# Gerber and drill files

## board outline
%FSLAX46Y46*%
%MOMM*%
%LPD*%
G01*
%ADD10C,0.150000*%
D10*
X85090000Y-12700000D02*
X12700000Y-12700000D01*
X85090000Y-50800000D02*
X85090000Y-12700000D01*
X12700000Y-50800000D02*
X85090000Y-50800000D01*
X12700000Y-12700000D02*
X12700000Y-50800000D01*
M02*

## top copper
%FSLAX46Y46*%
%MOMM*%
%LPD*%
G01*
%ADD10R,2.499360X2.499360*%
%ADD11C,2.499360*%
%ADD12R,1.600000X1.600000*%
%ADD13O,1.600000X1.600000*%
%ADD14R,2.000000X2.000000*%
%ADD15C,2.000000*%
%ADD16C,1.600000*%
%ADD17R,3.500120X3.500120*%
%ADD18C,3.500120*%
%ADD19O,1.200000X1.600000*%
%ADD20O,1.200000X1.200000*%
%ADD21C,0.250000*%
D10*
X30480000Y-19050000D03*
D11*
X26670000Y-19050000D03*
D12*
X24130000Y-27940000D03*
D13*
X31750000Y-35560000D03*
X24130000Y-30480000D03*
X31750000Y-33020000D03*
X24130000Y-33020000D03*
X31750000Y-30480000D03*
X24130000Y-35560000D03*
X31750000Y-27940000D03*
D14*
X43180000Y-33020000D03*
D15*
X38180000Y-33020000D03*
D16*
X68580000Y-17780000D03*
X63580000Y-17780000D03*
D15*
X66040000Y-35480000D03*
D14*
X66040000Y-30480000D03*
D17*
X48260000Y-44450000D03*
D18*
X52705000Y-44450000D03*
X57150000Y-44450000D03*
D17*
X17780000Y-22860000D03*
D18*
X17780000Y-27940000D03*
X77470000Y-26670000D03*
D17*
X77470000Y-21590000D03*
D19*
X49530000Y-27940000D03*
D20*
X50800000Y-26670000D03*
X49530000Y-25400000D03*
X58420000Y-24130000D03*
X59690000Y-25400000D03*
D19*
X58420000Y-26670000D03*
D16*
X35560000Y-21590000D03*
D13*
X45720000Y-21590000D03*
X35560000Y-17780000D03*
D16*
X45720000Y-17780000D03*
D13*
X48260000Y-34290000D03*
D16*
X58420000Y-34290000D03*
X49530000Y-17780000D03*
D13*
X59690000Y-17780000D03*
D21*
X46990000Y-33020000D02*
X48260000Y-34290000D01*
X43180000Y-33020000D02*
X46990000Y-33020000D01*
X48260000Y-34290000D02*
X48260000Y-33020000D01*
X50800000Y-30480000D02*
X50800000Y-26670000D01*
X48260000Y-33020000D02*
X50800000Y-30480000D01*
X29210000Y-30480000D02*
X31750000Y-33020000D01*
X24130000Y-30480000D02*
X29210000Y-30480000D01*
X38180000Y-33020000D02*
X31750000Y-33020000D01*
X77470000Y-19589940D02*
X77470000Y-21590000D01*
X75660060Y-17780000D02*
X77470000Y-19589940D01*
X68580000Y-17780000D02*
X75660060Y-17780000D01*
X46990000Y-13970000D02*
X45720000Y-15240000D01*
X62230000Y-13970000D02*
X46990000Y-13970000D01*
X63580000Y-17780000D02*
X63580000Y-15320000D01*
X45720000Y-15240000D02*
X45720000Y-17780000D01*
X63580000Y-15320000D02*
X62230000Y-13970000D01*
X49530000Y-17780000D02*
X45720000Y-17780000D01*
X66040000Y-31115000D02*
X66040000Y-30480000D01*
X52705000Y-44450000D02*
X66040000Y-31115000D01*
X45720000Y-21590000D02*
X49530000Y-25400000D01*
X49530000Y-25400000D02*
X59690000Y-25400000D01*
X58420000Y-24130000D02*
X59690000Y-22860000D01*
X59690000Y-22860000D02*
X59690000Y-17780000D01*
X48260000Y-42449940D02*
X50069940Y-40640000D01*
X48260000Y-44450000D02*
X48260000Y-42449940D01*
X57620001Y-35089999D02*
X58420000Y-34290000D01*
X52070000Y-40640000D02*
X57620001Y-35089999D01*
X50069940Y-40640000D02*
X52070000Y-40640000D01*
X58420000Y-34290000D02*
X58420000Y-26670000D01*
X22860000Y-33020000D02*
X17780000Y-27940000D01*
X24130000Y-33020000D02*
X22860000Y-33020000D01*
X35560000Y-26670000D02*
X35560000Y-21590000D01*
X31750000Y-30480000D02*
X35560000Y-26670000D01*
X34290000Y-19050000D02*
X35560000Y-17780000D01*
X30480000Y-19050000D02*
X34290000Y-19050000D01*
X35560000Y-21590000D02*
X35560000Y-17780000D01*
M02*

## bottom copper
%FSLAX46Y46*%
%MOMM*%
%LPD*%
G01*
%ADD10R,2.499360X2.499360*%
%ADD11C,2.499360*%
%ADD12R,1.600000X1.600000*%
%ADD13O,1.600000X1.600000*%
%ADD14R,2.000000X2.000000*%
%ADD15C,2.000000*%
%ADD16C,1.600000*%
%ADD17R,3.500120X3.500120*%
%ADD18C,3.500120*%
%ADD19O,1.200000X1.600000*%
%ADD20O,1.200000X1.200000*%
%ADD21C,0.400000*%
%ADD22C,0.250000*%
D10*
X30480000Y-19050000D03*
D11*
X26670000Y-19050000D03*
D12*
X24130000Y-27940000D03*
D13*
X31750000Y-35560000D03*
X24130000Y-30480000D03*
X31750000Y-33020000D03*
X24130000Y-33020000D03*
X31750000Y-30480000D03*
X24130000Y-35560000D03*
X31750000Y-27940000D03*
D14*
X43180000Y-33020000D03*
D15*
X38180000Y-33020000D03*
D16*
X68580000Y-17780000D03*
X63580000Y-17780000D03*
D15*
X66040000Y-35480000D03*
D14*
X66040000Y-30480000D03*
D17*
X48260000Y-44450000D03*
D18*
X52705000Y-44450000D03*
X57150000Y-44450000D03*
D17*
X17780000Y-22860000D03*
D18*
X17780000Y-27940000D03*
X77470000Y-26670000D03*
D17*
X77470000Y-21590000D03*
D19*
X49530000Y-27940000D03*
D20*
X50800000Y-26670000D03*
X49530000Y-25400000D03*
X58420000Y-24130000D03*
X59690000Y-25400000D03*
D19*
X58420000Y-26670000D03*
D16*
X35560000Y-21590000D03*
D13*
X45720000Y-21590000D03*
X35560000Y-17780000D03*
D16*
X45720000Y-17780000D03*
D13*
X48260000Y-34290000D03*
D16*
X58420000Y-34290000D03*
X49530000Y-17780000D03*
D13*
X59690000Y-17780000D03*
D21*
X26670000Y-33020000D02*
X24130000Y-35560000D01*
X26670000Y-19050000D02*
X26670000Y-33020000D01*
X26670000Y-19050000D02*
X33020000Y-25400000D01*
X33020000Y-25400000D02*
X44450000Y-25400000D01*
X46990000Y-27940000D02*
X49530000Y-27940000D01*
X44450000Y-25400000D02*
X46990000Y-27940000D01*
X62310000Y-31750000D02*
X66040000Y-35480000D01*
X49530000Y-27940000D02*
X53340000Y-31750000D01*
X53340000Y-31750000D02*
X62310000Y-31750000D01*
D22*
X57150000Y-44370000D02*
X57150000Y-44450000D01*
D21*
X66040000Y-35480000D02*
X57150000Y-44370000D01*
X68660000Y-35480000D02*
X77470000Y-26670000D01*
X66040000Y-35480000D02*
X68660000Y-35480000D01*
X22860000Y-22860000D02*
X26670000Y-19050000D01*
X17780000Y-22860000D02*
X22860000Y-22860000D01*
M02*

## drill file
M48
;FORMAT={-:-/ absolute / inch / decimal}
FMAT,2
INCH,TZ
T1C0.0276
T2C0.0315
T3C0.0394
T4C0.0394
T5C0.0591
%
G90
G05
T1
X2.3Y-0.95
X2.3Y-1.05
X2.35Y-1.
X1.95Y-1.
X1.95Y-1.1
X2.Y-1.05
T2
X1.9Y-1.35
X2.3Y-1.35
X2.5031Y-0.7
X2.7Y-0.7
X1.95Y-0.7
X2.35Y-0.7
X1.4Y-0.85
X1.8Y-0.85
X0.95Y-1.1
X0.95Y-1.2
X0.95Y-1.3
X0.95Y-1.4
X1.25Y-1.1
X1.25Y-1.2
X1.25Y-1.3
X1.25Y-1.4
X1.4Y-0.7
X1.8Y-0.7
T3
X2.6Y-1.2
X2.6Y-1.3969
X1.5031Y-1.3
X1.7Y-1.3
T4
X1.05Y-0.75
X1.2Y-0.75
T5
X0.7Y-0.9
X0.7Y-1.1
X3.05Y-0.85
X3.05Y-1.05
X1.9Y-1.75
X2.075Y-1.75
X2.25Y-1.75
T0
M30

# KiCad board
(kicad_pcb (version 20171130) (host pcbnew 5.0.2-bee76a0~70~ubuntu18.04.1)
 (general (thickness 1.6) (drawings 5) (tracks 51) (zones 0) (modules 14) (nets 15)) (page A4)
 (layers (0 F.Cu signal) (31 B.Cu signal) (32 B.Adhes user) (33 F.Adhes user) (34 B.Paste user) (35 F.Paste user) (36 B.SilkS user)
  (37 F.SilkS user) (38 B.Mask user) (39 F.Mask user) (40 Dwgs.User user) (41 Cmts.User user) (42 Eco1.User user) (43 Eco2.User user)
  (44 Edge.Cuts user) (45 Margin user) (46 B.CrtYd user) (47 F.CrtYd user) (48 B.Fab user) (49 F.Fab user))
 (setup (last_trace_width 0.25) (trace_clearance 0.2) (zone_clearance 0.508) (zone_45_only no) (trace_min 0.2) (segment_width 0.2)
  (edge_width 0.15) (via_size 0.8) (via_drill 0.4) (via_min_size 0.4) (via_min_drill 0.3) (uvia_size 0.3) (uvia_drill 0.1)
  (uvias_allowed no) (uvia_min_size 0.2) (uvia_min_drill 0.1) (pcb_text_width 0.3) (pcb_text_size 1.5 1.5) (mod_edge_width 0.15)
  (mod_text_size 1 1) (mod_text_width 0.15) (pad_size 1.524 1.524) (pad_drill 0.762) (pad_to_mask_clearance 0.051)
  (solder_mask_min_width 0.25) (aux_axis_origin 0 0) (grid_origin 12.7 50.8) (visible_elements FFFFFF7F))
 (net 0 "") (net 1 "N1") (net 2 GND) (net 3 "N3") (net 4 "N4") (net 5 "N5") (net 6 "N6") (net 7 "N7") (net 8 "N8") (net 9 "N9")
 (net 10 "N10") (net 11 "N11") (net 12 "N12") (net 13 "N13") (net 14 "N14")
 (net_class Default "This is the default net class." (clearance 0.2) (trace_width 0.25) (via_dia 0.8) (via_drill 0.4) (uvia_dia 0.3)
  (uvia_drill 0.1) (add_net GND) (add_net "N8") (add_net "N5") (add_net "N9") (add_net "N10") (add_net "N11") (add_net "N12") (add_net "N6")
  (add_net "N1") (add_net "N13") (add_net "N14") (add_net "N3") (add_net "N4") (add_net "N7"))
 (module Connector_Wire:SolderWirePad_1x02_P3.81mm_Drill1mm (layer F.Cu) (at 30.48 19.05 180)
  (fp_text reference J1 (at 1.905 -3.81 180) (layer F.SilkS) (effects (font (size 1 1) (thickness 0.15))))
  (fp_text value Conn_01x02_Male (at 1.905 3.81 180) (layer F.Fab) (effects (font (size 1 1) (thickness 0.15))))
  (pad 1 thru_hole rect (at 0 0 180) (size 2.49936 2.49936) (drill 1.00076) (layers *.Cu *.Mask) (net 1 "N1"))
  (pad 2 thru_hole circle (at 3.81 0 180) (size 2.49936 2.49936) (drill 1.00076) (layers *.Cu *.Mask) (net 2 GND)))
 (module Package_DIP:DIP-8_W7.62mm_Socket (layer F.Cu) (at 24.13 27.94)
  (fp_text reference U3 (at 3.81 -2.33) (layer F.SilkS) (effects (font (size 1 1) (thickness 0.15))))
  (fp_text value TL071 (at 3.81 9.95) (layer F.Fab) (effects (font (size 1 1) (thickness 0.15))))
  (pad 1 thru_hole rect (at 0 0) (size 1.6 1.6) (drill 0.8) (layers *.Cu *.Mask) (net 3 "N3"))
  (pad 5 thru_hole oval (at 7.62 7.62) (size 1.6 1.6) (drill 0.8) (layers *.Cu *.Mask) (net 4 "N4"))
  (pad 2 thru_hole oval (at 0 2.54) (size 1.6 1.6) (drill 0.8) (layers *.Cu *.Mask) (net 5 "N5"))
  (pad 6 thru_hole oval (at 7.62 5.08) (size 1.6 1.6) (drill 0.8) (layers *.Cu *.Mask) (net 5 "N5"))
  (pad 3 thru_hole oval (at 0 5.08) (size 1.6 1.6) (drill 0.8) (layers *.Cu *.Mask) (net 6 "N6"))
  (pad 7 thru_hole oval (at 7.62 2.54) (size 1.6 1.6) (drill 0.8) (layers *.Cu *.Mask) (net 1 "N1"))
  (pad 4 thru_hole oval (at 0 7.62) (size 1.6 1.6) (drill 0.8) (layers *.Cu *.Mask) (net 2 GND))
  (pad 8 thru_hole oval (at 7.62 0) (size 1.6 1.6) (drill 0.8) (layers *.Cu *.Mask) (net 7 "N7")))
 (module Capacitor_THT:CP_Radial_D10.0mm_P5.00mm (layer F.Cu) (at 43.18 33.02 180)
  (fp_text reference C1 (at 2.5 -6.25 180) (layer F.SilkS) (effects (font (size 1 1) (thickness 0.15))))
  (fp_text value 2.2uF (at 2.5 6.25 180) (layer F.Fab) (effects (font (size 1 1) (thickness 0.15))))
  (pad 1 thru_hole rect (at 0 0 180) (size 2 2) (drill 1) (layers *.Cu *.Mask) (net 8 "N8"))
  (pad 2 thru_hole circle (at 5 0 180) (size 2 2) (drill 1) (layers *.Cu *.Mask) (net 5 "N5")))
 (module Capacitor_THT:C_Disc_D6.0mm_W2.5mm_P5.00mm (layer F.Cu) (at 68.58 17.78 180)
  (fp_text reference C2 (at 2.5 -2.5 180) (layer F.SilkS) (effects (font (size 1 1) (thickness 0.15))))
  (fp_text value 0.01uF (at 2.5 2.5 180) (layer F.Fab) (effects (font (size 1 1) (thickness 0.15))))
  (pad 1 thru_hole circle (at 0 0 180) (size 1.6 1.6) (drill 0.8) (layers *.Cu *.Mask) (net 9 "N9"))
  (pad 2 thru_hole circle (at 5 0 180) (size 1.6 1.6) (drill 0.8) (layers *.Cu *.Mask) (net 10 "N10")))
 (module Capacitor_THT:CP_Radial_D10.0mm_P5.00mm (layer F.Cu) (at 66.04 30.48 270)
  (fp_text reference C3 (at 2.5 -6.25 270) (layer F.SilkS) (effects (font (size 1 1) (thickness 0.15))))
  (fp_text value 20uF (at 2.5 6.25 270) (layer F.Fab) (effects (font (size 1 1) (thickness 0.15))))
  (pad 2 thru_hole circle (at 5 0 270) (size 2 2) (drill 1) (layers *.Cu *.Mask) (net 2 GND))
  (pad 1 thru_hole rect (at 0 0 270) (size 2 2) (drill 1) (layers *.Cu *.Mask) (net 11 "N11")))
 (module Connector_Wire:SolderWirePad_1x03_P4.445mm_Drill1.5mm (layer F.Cu) (at 48.26 44.45)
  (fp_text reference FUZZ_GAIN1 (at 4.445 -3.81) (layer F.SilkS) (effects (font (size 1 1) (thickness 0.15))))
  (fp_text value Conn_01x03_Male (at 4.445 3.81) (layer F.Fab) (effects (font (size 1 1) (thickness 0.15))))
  (pad 1 thru_hole rect (at 0 0) (size 3.50012 3.50012) (drill 1.50114) (layers *.Cu *.Mask) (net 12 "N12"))
  (pad 2 thru_hole circle (at 4.445 0) (size 3.50012 3.50012) (drill 1.50114) (layers *.Cu *.Mask) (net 11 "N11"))
  (pad 3 thru_hole circle (at 8.89 0) (size 3.50012 3.50012) (drill 1.50114) (layers *.Cu *.Mask) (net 2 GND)))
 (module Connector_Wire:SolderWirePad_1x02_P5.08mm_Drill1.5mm (layer F.Cu) (at 17.78 22.86 270)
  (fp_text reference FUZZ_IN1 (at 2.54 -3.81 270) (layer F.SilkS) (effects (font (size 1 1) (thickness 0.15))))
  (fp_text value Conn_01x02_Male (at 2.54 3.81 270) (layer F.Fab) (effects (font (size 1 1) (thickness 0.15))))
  (pad 1 thru_hole rect (at 0 0 270) (size 3.50012 3.50012) (drill 1.50114) (layers *.Cu *.Mask) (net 2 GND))
  (pad 2 thru_hole circle (at 5.08 0 270) (size 3.50012 3.50012) (drill 1.50114) (layers *.Cu *.Mask) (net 6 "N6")))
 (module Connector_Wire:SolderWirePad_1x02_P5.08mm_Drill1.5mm (layer F.Cu) (at 77.47 21.59 270)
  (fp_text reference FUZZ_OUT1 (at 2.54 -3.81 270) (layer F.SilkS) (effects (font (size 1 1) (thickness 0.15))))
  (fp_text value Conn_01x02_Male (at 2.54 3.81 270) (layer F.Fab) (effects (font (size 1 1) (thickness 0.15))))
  (pad 2 thru_hole circle (at 5.08 0 270) (size 3.50012 3.50012) (drill 1.50114) (layers *.Cu *.Mask) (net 2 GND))
  (pad 1 thru_hole rect (at 0 0 270) (size 3.50012 3.50012) (drill 1.50114) (layers *.Cu *.Mask) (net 9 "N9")))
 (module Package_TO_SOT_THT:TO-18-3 (layer F.Cu) (at 49.53 27.94 90)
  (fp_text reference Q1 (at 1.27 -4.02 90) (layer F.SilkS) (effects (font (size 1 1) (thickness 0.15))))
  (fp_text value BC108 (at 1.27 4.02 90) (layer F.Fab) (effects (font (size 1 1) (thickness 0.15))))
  (pad 1 thru_hole oval (at 0 0 90) (size 1.6 1.2) (drill 0.7) (layers *.Cu *.Mask) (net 2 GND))
  (pad 2 thru_hole oval (at 1.27 1.27 90) (size 1.2 1.2) (drill 0.7) (layers *.Cu *.Mask) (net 8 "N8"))
  (pad 3 thru_hole oval (at 2.54 0 90) (size 1.2 1.2) (drill 0.7) (layers *.Cu *.Mask) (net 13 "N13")))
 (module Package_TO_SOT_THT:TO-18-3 (layer F.Cu) (at 58.42 26.67 90)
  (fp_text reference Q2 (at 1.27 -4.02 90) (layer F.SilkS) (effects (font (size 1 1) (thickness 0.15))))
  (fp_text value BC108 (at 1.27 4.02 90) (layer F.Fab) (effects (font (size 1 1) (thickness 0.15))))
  (pad 3 thru_hole oval (at 2.54 0 90) (size 1.2 1.2) (drill 0.7) (layers *.Cu *.Mask) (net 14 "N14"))
  (pad 2 thru_hole oval (at 1.27 1.27 90) (size 1.2 1.2) (drill 0.7) (layers *.Cu *.Mask) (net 13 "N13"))
  (pad 1 thru_hole oval (at 0 0 90) (size 1.6 1.2) (drill 0.7) (layers *.Cu *.Mask) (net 12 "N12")))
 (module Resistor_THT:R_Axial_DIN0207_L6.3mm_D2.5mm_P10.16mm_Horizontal (layer F.Cu) (at 35.56 21.59)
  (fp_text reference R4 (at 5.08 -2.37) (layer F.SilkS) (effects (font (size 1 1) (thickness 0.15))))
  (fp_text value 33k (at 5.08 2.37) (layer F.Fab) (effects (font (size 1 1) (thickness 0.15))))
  (pad 1 thru_hole circle (at 0 0) (size 1.6 1.6) (drill 0.8) (layers *.Cu *.Mask) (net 1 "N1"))
  (pad 2 thru_hole oval (at 10.16 0) (size 1.6 1.6) (drill 0.8) (layers *.Cu *.Mask) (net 13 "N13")))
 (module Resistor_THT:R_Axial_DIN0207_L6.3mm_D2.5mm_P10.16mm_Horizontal (layer F.Cu) (at 45.72 17.78 180)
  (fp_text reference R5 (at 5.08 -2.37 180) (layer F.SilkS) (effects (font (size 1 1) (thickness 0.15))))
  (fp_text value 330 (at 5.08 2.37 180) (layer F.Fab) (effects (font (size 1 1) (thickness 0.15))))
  (pad 2 thru_hole oval (at 10.16 0 180) (size 1.6 1.6) (drill 0.8) (layers *.Cu *.Mask) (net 1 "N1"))
  (pad 1 thru_hole circle (at 0 0 180) (size 1.6 1.6) (drill 0.8) (layers *.Cu *.Mask) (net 10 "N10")))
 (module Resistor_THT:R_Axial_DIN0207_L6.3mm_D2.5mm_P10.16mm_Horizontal (layer F.Cu) (at 58.42 34.29 180)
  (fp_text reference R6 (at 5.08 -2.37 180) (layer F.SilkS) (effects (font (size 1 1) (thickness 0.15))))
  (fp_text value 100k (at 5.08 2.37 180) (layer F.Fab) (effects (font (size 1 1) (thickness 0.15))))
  (pad 2 thru_hole oval (at 10.16 0 180) (size 1.6 1.6) (drill 0.8) (layers *.Cu *.Mask) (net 8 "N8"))
  (pad 1 thru_hole circle (at 0 0 180) (size 1.6 1.6) (drill 0.8) (layers *.Cu *.Mask) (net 12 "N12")))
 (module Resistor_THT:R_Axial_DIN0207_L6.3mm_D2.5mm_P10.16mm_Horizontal (layer F.Cu) (at 49.53 17.78)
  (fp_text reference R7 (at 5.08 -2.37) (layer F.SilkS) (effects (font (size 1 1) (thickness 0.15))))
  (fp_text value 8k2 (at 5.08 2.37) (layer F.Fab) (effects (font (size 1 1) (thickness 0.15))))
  (pad 1 thru_hole circle (at 0 0) (size 1.6 1.6) (drill 0.8) (layers *.Cu *.Mask) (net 10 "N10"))
  (pad 2 thru_hole oval (at 10.16 0) (size 1.6 1.6) (drill 0.8) (layers *.Cu *.Mask) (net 14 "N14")))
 (gr_line (start 85.09 12.7) (end 12.7 12.7) (layer Edge.Cuts) (width 0.15))
 (gr_line (start 85.09 50.8) (end 85.09 12.7) (layer Edge.Cuts) (width 0.15))
 (gr_line (start 12.7 50.8) (end 85.09 50.8) (layer Edge.Cuts) (width 0.15))
 (gr_line (start 12.7 12.7) (end 12.7 50.8) (layer Edge.Cuts) (width 0.15))
 (segment (start 46.99 33.02) (end 48.26 34.29) (width 0.25) (layer F.Cu) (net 8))
 (segment (start 43.18 33.02) (end 46.99 33.02) (width 0.25) (layer F.Cu) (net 8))
 (segment (start 48.26 34.29) (end 48.26 33.02) (width 0.25) (layer F.Cu) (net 8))
 (segment (start 50.8 30.48) (end 50.8 26.67) (width 0.25) (layer F.Cu) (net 8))
 (segment (start 48.26 33.02) (end 50.8 30.48) (width 0.25) (layer F.Cu) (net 8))
 (segment (start 29.21 30.48) (end 31.75 33.02) (width 0.25) (layer F.Cu) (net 5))
 (segment (start 24.13 30.48) (end 29.21 30.48) (width 0.25) (layer F.Cu) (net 5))
 (segment (start 38.18 33.02) (end 31.75 33.02) (width 0.25) (layer F.Cu) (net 5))
 (segment (start 77.47 19.58994) (end 77.47 21.59) (width 0.25) (layer F.Cu) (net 9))
 (segment (start 75.66006 17.78) (end 77.47 19.58994) (width 0.25) (layer F.Cu) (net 9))
 (segment (start 68.58 17.78) (end 75.66006 17.78) (width 0.25) (layer F.Cu) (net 9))
 (segment (start 46.99 13.97) (end 45.72 15.24) (width 0.25) (layer F.Cu) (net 10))
 (segment (start 62.23 13.97) (end 46.99 13.97) (width 0.25) (layer F.Cu) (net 10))
 (segment (start 63.58 17.78) (end 63.58 15.32) (width 0.25) (layer F.Cu) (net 10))
 (segment (start 45.72 15.24) (end 45.72 17.78) (width 0.25) (layer F.Cu) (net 10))
 (segment (start 63.58 15.32) (end 62.23 13.97) (width 0.25) (layer F.Cu) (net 10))
 (segment (start 49.53 17.78) (end 45.72 17.78) (width 0.25) (layer F.Cu) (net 10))
 (segment (start 26.67 33.02) (end 24.13 35.56) (width 0.4) (layer B.Cu) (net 2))
 (segment (start 26.67 19.05) (end 26.67 33.02) (width 0.4) (layer B.Cu) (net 2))
 (segment (start 26.67 19.05) (end 33.02 25.4) (width 0.4) (layer B.Cu) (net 2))
 (segment (start 33.02 25.4) (end 44.45 25.4) (width 0.4) (layer B.Cu) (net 2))
 (segment (start 46.99 27.94) (end 49.53 27.94) (width 0.4) (layer B.Cu) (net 2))
 (segment (start 44.45 25.4) (end 46.99 27.94) (width 0.4) (layer B.Cu) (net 2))
 (segment (start 62.31 31.75) (end 66.04 35.48) (width 0.4) (layer B.Cu) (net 2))
 (segment (start 49.53 27.94) (end 53.34 31.75) (width 0.4) (layer B.Cu) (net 2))
 (segment (start 53.34 31.75) (end 62.31 31.75) (width 0.4) (layer B.Cu) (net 2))
 (segment (start 57.15 44.37) (end 57.15 44.45) (width 0.25) (layer B.Cu) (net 2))
 (segment (start 66.04 35.48) (end 57.15 44.37) (width 0.4) (layer B.Cu) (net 2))
 (segment (start 68.66 35.48) (end 77.47 26.67) (width 0.4) (layer B.Cu) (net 2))
 (segment (start 66.04 35.48) (end 68.66 35.48) (width 0.4) (layer B.Cu) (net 2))
 (segment (start 22.86 22.86) (end 26.67 19.05) (width 0.4) (layer B.Cu) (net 2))
 (segment (start 17.78 22.86) (end 22.86 22.86) (width 0.4) (layer B.Cu) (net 2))
 (segment (start 66.04 31.115) (end 66.04 30.48) (width 0.25) (layer F.Cu) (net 11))
 (segment (start 52.705 44.45) (end 66.04 31.115) (width 0.25) (layer F.Cu) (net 11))
 (segment (start 45.72 21.59) (end 49.53 25.4) (width 0.25) (layer F.Cu) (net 13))
 (segment (start 49.53 25.4) (end 59.69 25.4) (width 0.25) (layer F.Cu) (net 13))
 (segment (start 58.42 24.13) (end 59.69 22.86) (width 0.25) (layer F.Cu) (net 14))
 (segment (start 59.69 22.86) (end 59.69 17.78) (width 0.25) (layer F.Cu) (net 14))
 (segment (start 48.26 42.44994) (end 50.06994 40.64) (width 0.25) (layer F.Cu) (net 12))
 (segment (start 48.26 44.45) (end 48.26 42.44994) (width 0.25) (layer F.Cu) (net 12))
 (segment (start 57.620001 35.089999) (end 58.42 34.29) (width 0.25) (layer F.Cu) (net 12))
 (segment (start 52.07 40.64) (end 57.620001 35.089999) (width 0.25) (layer F.Cu) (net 12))
 (segment (start 50.06994 40.64) (end 52.07 40.64) (width 0.25) (layer F.Cu) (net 12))
 (segment (start 58.42 34.29) (end 58.42 26.67) (width 0.25) (layer F.Cu) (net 12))
 (segment (start 22.86 33.02) (end 17.78 27.94) (width 0.25) (layer F.Cu) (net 6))
 (segment (start 24.13 33.02) (end 22.86 33.02) (width 0.25) (layer F.Cu) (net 6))
 (segment (start 35.56 26.67) (end 35.56 21.59) (width 0.25) (layer F.Cu) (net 1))
 (segment (start 31.75 30.48) (end 35.56 26.67) (width 0.25) (layer F.Cu) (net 1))
 (segment (start 34.29 19.05) (end 35.56 17.78) (width 0.25) (layer F.Cu) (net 1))
 (segment (start 30.48 19.05) (end 34.29 19.05) (width 0.25) (layer F.Cu) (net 1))
 (segment (start 35.56 21.59) (end 35.56 17.78) (width 0.25) (layer F.Cu) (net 1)))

